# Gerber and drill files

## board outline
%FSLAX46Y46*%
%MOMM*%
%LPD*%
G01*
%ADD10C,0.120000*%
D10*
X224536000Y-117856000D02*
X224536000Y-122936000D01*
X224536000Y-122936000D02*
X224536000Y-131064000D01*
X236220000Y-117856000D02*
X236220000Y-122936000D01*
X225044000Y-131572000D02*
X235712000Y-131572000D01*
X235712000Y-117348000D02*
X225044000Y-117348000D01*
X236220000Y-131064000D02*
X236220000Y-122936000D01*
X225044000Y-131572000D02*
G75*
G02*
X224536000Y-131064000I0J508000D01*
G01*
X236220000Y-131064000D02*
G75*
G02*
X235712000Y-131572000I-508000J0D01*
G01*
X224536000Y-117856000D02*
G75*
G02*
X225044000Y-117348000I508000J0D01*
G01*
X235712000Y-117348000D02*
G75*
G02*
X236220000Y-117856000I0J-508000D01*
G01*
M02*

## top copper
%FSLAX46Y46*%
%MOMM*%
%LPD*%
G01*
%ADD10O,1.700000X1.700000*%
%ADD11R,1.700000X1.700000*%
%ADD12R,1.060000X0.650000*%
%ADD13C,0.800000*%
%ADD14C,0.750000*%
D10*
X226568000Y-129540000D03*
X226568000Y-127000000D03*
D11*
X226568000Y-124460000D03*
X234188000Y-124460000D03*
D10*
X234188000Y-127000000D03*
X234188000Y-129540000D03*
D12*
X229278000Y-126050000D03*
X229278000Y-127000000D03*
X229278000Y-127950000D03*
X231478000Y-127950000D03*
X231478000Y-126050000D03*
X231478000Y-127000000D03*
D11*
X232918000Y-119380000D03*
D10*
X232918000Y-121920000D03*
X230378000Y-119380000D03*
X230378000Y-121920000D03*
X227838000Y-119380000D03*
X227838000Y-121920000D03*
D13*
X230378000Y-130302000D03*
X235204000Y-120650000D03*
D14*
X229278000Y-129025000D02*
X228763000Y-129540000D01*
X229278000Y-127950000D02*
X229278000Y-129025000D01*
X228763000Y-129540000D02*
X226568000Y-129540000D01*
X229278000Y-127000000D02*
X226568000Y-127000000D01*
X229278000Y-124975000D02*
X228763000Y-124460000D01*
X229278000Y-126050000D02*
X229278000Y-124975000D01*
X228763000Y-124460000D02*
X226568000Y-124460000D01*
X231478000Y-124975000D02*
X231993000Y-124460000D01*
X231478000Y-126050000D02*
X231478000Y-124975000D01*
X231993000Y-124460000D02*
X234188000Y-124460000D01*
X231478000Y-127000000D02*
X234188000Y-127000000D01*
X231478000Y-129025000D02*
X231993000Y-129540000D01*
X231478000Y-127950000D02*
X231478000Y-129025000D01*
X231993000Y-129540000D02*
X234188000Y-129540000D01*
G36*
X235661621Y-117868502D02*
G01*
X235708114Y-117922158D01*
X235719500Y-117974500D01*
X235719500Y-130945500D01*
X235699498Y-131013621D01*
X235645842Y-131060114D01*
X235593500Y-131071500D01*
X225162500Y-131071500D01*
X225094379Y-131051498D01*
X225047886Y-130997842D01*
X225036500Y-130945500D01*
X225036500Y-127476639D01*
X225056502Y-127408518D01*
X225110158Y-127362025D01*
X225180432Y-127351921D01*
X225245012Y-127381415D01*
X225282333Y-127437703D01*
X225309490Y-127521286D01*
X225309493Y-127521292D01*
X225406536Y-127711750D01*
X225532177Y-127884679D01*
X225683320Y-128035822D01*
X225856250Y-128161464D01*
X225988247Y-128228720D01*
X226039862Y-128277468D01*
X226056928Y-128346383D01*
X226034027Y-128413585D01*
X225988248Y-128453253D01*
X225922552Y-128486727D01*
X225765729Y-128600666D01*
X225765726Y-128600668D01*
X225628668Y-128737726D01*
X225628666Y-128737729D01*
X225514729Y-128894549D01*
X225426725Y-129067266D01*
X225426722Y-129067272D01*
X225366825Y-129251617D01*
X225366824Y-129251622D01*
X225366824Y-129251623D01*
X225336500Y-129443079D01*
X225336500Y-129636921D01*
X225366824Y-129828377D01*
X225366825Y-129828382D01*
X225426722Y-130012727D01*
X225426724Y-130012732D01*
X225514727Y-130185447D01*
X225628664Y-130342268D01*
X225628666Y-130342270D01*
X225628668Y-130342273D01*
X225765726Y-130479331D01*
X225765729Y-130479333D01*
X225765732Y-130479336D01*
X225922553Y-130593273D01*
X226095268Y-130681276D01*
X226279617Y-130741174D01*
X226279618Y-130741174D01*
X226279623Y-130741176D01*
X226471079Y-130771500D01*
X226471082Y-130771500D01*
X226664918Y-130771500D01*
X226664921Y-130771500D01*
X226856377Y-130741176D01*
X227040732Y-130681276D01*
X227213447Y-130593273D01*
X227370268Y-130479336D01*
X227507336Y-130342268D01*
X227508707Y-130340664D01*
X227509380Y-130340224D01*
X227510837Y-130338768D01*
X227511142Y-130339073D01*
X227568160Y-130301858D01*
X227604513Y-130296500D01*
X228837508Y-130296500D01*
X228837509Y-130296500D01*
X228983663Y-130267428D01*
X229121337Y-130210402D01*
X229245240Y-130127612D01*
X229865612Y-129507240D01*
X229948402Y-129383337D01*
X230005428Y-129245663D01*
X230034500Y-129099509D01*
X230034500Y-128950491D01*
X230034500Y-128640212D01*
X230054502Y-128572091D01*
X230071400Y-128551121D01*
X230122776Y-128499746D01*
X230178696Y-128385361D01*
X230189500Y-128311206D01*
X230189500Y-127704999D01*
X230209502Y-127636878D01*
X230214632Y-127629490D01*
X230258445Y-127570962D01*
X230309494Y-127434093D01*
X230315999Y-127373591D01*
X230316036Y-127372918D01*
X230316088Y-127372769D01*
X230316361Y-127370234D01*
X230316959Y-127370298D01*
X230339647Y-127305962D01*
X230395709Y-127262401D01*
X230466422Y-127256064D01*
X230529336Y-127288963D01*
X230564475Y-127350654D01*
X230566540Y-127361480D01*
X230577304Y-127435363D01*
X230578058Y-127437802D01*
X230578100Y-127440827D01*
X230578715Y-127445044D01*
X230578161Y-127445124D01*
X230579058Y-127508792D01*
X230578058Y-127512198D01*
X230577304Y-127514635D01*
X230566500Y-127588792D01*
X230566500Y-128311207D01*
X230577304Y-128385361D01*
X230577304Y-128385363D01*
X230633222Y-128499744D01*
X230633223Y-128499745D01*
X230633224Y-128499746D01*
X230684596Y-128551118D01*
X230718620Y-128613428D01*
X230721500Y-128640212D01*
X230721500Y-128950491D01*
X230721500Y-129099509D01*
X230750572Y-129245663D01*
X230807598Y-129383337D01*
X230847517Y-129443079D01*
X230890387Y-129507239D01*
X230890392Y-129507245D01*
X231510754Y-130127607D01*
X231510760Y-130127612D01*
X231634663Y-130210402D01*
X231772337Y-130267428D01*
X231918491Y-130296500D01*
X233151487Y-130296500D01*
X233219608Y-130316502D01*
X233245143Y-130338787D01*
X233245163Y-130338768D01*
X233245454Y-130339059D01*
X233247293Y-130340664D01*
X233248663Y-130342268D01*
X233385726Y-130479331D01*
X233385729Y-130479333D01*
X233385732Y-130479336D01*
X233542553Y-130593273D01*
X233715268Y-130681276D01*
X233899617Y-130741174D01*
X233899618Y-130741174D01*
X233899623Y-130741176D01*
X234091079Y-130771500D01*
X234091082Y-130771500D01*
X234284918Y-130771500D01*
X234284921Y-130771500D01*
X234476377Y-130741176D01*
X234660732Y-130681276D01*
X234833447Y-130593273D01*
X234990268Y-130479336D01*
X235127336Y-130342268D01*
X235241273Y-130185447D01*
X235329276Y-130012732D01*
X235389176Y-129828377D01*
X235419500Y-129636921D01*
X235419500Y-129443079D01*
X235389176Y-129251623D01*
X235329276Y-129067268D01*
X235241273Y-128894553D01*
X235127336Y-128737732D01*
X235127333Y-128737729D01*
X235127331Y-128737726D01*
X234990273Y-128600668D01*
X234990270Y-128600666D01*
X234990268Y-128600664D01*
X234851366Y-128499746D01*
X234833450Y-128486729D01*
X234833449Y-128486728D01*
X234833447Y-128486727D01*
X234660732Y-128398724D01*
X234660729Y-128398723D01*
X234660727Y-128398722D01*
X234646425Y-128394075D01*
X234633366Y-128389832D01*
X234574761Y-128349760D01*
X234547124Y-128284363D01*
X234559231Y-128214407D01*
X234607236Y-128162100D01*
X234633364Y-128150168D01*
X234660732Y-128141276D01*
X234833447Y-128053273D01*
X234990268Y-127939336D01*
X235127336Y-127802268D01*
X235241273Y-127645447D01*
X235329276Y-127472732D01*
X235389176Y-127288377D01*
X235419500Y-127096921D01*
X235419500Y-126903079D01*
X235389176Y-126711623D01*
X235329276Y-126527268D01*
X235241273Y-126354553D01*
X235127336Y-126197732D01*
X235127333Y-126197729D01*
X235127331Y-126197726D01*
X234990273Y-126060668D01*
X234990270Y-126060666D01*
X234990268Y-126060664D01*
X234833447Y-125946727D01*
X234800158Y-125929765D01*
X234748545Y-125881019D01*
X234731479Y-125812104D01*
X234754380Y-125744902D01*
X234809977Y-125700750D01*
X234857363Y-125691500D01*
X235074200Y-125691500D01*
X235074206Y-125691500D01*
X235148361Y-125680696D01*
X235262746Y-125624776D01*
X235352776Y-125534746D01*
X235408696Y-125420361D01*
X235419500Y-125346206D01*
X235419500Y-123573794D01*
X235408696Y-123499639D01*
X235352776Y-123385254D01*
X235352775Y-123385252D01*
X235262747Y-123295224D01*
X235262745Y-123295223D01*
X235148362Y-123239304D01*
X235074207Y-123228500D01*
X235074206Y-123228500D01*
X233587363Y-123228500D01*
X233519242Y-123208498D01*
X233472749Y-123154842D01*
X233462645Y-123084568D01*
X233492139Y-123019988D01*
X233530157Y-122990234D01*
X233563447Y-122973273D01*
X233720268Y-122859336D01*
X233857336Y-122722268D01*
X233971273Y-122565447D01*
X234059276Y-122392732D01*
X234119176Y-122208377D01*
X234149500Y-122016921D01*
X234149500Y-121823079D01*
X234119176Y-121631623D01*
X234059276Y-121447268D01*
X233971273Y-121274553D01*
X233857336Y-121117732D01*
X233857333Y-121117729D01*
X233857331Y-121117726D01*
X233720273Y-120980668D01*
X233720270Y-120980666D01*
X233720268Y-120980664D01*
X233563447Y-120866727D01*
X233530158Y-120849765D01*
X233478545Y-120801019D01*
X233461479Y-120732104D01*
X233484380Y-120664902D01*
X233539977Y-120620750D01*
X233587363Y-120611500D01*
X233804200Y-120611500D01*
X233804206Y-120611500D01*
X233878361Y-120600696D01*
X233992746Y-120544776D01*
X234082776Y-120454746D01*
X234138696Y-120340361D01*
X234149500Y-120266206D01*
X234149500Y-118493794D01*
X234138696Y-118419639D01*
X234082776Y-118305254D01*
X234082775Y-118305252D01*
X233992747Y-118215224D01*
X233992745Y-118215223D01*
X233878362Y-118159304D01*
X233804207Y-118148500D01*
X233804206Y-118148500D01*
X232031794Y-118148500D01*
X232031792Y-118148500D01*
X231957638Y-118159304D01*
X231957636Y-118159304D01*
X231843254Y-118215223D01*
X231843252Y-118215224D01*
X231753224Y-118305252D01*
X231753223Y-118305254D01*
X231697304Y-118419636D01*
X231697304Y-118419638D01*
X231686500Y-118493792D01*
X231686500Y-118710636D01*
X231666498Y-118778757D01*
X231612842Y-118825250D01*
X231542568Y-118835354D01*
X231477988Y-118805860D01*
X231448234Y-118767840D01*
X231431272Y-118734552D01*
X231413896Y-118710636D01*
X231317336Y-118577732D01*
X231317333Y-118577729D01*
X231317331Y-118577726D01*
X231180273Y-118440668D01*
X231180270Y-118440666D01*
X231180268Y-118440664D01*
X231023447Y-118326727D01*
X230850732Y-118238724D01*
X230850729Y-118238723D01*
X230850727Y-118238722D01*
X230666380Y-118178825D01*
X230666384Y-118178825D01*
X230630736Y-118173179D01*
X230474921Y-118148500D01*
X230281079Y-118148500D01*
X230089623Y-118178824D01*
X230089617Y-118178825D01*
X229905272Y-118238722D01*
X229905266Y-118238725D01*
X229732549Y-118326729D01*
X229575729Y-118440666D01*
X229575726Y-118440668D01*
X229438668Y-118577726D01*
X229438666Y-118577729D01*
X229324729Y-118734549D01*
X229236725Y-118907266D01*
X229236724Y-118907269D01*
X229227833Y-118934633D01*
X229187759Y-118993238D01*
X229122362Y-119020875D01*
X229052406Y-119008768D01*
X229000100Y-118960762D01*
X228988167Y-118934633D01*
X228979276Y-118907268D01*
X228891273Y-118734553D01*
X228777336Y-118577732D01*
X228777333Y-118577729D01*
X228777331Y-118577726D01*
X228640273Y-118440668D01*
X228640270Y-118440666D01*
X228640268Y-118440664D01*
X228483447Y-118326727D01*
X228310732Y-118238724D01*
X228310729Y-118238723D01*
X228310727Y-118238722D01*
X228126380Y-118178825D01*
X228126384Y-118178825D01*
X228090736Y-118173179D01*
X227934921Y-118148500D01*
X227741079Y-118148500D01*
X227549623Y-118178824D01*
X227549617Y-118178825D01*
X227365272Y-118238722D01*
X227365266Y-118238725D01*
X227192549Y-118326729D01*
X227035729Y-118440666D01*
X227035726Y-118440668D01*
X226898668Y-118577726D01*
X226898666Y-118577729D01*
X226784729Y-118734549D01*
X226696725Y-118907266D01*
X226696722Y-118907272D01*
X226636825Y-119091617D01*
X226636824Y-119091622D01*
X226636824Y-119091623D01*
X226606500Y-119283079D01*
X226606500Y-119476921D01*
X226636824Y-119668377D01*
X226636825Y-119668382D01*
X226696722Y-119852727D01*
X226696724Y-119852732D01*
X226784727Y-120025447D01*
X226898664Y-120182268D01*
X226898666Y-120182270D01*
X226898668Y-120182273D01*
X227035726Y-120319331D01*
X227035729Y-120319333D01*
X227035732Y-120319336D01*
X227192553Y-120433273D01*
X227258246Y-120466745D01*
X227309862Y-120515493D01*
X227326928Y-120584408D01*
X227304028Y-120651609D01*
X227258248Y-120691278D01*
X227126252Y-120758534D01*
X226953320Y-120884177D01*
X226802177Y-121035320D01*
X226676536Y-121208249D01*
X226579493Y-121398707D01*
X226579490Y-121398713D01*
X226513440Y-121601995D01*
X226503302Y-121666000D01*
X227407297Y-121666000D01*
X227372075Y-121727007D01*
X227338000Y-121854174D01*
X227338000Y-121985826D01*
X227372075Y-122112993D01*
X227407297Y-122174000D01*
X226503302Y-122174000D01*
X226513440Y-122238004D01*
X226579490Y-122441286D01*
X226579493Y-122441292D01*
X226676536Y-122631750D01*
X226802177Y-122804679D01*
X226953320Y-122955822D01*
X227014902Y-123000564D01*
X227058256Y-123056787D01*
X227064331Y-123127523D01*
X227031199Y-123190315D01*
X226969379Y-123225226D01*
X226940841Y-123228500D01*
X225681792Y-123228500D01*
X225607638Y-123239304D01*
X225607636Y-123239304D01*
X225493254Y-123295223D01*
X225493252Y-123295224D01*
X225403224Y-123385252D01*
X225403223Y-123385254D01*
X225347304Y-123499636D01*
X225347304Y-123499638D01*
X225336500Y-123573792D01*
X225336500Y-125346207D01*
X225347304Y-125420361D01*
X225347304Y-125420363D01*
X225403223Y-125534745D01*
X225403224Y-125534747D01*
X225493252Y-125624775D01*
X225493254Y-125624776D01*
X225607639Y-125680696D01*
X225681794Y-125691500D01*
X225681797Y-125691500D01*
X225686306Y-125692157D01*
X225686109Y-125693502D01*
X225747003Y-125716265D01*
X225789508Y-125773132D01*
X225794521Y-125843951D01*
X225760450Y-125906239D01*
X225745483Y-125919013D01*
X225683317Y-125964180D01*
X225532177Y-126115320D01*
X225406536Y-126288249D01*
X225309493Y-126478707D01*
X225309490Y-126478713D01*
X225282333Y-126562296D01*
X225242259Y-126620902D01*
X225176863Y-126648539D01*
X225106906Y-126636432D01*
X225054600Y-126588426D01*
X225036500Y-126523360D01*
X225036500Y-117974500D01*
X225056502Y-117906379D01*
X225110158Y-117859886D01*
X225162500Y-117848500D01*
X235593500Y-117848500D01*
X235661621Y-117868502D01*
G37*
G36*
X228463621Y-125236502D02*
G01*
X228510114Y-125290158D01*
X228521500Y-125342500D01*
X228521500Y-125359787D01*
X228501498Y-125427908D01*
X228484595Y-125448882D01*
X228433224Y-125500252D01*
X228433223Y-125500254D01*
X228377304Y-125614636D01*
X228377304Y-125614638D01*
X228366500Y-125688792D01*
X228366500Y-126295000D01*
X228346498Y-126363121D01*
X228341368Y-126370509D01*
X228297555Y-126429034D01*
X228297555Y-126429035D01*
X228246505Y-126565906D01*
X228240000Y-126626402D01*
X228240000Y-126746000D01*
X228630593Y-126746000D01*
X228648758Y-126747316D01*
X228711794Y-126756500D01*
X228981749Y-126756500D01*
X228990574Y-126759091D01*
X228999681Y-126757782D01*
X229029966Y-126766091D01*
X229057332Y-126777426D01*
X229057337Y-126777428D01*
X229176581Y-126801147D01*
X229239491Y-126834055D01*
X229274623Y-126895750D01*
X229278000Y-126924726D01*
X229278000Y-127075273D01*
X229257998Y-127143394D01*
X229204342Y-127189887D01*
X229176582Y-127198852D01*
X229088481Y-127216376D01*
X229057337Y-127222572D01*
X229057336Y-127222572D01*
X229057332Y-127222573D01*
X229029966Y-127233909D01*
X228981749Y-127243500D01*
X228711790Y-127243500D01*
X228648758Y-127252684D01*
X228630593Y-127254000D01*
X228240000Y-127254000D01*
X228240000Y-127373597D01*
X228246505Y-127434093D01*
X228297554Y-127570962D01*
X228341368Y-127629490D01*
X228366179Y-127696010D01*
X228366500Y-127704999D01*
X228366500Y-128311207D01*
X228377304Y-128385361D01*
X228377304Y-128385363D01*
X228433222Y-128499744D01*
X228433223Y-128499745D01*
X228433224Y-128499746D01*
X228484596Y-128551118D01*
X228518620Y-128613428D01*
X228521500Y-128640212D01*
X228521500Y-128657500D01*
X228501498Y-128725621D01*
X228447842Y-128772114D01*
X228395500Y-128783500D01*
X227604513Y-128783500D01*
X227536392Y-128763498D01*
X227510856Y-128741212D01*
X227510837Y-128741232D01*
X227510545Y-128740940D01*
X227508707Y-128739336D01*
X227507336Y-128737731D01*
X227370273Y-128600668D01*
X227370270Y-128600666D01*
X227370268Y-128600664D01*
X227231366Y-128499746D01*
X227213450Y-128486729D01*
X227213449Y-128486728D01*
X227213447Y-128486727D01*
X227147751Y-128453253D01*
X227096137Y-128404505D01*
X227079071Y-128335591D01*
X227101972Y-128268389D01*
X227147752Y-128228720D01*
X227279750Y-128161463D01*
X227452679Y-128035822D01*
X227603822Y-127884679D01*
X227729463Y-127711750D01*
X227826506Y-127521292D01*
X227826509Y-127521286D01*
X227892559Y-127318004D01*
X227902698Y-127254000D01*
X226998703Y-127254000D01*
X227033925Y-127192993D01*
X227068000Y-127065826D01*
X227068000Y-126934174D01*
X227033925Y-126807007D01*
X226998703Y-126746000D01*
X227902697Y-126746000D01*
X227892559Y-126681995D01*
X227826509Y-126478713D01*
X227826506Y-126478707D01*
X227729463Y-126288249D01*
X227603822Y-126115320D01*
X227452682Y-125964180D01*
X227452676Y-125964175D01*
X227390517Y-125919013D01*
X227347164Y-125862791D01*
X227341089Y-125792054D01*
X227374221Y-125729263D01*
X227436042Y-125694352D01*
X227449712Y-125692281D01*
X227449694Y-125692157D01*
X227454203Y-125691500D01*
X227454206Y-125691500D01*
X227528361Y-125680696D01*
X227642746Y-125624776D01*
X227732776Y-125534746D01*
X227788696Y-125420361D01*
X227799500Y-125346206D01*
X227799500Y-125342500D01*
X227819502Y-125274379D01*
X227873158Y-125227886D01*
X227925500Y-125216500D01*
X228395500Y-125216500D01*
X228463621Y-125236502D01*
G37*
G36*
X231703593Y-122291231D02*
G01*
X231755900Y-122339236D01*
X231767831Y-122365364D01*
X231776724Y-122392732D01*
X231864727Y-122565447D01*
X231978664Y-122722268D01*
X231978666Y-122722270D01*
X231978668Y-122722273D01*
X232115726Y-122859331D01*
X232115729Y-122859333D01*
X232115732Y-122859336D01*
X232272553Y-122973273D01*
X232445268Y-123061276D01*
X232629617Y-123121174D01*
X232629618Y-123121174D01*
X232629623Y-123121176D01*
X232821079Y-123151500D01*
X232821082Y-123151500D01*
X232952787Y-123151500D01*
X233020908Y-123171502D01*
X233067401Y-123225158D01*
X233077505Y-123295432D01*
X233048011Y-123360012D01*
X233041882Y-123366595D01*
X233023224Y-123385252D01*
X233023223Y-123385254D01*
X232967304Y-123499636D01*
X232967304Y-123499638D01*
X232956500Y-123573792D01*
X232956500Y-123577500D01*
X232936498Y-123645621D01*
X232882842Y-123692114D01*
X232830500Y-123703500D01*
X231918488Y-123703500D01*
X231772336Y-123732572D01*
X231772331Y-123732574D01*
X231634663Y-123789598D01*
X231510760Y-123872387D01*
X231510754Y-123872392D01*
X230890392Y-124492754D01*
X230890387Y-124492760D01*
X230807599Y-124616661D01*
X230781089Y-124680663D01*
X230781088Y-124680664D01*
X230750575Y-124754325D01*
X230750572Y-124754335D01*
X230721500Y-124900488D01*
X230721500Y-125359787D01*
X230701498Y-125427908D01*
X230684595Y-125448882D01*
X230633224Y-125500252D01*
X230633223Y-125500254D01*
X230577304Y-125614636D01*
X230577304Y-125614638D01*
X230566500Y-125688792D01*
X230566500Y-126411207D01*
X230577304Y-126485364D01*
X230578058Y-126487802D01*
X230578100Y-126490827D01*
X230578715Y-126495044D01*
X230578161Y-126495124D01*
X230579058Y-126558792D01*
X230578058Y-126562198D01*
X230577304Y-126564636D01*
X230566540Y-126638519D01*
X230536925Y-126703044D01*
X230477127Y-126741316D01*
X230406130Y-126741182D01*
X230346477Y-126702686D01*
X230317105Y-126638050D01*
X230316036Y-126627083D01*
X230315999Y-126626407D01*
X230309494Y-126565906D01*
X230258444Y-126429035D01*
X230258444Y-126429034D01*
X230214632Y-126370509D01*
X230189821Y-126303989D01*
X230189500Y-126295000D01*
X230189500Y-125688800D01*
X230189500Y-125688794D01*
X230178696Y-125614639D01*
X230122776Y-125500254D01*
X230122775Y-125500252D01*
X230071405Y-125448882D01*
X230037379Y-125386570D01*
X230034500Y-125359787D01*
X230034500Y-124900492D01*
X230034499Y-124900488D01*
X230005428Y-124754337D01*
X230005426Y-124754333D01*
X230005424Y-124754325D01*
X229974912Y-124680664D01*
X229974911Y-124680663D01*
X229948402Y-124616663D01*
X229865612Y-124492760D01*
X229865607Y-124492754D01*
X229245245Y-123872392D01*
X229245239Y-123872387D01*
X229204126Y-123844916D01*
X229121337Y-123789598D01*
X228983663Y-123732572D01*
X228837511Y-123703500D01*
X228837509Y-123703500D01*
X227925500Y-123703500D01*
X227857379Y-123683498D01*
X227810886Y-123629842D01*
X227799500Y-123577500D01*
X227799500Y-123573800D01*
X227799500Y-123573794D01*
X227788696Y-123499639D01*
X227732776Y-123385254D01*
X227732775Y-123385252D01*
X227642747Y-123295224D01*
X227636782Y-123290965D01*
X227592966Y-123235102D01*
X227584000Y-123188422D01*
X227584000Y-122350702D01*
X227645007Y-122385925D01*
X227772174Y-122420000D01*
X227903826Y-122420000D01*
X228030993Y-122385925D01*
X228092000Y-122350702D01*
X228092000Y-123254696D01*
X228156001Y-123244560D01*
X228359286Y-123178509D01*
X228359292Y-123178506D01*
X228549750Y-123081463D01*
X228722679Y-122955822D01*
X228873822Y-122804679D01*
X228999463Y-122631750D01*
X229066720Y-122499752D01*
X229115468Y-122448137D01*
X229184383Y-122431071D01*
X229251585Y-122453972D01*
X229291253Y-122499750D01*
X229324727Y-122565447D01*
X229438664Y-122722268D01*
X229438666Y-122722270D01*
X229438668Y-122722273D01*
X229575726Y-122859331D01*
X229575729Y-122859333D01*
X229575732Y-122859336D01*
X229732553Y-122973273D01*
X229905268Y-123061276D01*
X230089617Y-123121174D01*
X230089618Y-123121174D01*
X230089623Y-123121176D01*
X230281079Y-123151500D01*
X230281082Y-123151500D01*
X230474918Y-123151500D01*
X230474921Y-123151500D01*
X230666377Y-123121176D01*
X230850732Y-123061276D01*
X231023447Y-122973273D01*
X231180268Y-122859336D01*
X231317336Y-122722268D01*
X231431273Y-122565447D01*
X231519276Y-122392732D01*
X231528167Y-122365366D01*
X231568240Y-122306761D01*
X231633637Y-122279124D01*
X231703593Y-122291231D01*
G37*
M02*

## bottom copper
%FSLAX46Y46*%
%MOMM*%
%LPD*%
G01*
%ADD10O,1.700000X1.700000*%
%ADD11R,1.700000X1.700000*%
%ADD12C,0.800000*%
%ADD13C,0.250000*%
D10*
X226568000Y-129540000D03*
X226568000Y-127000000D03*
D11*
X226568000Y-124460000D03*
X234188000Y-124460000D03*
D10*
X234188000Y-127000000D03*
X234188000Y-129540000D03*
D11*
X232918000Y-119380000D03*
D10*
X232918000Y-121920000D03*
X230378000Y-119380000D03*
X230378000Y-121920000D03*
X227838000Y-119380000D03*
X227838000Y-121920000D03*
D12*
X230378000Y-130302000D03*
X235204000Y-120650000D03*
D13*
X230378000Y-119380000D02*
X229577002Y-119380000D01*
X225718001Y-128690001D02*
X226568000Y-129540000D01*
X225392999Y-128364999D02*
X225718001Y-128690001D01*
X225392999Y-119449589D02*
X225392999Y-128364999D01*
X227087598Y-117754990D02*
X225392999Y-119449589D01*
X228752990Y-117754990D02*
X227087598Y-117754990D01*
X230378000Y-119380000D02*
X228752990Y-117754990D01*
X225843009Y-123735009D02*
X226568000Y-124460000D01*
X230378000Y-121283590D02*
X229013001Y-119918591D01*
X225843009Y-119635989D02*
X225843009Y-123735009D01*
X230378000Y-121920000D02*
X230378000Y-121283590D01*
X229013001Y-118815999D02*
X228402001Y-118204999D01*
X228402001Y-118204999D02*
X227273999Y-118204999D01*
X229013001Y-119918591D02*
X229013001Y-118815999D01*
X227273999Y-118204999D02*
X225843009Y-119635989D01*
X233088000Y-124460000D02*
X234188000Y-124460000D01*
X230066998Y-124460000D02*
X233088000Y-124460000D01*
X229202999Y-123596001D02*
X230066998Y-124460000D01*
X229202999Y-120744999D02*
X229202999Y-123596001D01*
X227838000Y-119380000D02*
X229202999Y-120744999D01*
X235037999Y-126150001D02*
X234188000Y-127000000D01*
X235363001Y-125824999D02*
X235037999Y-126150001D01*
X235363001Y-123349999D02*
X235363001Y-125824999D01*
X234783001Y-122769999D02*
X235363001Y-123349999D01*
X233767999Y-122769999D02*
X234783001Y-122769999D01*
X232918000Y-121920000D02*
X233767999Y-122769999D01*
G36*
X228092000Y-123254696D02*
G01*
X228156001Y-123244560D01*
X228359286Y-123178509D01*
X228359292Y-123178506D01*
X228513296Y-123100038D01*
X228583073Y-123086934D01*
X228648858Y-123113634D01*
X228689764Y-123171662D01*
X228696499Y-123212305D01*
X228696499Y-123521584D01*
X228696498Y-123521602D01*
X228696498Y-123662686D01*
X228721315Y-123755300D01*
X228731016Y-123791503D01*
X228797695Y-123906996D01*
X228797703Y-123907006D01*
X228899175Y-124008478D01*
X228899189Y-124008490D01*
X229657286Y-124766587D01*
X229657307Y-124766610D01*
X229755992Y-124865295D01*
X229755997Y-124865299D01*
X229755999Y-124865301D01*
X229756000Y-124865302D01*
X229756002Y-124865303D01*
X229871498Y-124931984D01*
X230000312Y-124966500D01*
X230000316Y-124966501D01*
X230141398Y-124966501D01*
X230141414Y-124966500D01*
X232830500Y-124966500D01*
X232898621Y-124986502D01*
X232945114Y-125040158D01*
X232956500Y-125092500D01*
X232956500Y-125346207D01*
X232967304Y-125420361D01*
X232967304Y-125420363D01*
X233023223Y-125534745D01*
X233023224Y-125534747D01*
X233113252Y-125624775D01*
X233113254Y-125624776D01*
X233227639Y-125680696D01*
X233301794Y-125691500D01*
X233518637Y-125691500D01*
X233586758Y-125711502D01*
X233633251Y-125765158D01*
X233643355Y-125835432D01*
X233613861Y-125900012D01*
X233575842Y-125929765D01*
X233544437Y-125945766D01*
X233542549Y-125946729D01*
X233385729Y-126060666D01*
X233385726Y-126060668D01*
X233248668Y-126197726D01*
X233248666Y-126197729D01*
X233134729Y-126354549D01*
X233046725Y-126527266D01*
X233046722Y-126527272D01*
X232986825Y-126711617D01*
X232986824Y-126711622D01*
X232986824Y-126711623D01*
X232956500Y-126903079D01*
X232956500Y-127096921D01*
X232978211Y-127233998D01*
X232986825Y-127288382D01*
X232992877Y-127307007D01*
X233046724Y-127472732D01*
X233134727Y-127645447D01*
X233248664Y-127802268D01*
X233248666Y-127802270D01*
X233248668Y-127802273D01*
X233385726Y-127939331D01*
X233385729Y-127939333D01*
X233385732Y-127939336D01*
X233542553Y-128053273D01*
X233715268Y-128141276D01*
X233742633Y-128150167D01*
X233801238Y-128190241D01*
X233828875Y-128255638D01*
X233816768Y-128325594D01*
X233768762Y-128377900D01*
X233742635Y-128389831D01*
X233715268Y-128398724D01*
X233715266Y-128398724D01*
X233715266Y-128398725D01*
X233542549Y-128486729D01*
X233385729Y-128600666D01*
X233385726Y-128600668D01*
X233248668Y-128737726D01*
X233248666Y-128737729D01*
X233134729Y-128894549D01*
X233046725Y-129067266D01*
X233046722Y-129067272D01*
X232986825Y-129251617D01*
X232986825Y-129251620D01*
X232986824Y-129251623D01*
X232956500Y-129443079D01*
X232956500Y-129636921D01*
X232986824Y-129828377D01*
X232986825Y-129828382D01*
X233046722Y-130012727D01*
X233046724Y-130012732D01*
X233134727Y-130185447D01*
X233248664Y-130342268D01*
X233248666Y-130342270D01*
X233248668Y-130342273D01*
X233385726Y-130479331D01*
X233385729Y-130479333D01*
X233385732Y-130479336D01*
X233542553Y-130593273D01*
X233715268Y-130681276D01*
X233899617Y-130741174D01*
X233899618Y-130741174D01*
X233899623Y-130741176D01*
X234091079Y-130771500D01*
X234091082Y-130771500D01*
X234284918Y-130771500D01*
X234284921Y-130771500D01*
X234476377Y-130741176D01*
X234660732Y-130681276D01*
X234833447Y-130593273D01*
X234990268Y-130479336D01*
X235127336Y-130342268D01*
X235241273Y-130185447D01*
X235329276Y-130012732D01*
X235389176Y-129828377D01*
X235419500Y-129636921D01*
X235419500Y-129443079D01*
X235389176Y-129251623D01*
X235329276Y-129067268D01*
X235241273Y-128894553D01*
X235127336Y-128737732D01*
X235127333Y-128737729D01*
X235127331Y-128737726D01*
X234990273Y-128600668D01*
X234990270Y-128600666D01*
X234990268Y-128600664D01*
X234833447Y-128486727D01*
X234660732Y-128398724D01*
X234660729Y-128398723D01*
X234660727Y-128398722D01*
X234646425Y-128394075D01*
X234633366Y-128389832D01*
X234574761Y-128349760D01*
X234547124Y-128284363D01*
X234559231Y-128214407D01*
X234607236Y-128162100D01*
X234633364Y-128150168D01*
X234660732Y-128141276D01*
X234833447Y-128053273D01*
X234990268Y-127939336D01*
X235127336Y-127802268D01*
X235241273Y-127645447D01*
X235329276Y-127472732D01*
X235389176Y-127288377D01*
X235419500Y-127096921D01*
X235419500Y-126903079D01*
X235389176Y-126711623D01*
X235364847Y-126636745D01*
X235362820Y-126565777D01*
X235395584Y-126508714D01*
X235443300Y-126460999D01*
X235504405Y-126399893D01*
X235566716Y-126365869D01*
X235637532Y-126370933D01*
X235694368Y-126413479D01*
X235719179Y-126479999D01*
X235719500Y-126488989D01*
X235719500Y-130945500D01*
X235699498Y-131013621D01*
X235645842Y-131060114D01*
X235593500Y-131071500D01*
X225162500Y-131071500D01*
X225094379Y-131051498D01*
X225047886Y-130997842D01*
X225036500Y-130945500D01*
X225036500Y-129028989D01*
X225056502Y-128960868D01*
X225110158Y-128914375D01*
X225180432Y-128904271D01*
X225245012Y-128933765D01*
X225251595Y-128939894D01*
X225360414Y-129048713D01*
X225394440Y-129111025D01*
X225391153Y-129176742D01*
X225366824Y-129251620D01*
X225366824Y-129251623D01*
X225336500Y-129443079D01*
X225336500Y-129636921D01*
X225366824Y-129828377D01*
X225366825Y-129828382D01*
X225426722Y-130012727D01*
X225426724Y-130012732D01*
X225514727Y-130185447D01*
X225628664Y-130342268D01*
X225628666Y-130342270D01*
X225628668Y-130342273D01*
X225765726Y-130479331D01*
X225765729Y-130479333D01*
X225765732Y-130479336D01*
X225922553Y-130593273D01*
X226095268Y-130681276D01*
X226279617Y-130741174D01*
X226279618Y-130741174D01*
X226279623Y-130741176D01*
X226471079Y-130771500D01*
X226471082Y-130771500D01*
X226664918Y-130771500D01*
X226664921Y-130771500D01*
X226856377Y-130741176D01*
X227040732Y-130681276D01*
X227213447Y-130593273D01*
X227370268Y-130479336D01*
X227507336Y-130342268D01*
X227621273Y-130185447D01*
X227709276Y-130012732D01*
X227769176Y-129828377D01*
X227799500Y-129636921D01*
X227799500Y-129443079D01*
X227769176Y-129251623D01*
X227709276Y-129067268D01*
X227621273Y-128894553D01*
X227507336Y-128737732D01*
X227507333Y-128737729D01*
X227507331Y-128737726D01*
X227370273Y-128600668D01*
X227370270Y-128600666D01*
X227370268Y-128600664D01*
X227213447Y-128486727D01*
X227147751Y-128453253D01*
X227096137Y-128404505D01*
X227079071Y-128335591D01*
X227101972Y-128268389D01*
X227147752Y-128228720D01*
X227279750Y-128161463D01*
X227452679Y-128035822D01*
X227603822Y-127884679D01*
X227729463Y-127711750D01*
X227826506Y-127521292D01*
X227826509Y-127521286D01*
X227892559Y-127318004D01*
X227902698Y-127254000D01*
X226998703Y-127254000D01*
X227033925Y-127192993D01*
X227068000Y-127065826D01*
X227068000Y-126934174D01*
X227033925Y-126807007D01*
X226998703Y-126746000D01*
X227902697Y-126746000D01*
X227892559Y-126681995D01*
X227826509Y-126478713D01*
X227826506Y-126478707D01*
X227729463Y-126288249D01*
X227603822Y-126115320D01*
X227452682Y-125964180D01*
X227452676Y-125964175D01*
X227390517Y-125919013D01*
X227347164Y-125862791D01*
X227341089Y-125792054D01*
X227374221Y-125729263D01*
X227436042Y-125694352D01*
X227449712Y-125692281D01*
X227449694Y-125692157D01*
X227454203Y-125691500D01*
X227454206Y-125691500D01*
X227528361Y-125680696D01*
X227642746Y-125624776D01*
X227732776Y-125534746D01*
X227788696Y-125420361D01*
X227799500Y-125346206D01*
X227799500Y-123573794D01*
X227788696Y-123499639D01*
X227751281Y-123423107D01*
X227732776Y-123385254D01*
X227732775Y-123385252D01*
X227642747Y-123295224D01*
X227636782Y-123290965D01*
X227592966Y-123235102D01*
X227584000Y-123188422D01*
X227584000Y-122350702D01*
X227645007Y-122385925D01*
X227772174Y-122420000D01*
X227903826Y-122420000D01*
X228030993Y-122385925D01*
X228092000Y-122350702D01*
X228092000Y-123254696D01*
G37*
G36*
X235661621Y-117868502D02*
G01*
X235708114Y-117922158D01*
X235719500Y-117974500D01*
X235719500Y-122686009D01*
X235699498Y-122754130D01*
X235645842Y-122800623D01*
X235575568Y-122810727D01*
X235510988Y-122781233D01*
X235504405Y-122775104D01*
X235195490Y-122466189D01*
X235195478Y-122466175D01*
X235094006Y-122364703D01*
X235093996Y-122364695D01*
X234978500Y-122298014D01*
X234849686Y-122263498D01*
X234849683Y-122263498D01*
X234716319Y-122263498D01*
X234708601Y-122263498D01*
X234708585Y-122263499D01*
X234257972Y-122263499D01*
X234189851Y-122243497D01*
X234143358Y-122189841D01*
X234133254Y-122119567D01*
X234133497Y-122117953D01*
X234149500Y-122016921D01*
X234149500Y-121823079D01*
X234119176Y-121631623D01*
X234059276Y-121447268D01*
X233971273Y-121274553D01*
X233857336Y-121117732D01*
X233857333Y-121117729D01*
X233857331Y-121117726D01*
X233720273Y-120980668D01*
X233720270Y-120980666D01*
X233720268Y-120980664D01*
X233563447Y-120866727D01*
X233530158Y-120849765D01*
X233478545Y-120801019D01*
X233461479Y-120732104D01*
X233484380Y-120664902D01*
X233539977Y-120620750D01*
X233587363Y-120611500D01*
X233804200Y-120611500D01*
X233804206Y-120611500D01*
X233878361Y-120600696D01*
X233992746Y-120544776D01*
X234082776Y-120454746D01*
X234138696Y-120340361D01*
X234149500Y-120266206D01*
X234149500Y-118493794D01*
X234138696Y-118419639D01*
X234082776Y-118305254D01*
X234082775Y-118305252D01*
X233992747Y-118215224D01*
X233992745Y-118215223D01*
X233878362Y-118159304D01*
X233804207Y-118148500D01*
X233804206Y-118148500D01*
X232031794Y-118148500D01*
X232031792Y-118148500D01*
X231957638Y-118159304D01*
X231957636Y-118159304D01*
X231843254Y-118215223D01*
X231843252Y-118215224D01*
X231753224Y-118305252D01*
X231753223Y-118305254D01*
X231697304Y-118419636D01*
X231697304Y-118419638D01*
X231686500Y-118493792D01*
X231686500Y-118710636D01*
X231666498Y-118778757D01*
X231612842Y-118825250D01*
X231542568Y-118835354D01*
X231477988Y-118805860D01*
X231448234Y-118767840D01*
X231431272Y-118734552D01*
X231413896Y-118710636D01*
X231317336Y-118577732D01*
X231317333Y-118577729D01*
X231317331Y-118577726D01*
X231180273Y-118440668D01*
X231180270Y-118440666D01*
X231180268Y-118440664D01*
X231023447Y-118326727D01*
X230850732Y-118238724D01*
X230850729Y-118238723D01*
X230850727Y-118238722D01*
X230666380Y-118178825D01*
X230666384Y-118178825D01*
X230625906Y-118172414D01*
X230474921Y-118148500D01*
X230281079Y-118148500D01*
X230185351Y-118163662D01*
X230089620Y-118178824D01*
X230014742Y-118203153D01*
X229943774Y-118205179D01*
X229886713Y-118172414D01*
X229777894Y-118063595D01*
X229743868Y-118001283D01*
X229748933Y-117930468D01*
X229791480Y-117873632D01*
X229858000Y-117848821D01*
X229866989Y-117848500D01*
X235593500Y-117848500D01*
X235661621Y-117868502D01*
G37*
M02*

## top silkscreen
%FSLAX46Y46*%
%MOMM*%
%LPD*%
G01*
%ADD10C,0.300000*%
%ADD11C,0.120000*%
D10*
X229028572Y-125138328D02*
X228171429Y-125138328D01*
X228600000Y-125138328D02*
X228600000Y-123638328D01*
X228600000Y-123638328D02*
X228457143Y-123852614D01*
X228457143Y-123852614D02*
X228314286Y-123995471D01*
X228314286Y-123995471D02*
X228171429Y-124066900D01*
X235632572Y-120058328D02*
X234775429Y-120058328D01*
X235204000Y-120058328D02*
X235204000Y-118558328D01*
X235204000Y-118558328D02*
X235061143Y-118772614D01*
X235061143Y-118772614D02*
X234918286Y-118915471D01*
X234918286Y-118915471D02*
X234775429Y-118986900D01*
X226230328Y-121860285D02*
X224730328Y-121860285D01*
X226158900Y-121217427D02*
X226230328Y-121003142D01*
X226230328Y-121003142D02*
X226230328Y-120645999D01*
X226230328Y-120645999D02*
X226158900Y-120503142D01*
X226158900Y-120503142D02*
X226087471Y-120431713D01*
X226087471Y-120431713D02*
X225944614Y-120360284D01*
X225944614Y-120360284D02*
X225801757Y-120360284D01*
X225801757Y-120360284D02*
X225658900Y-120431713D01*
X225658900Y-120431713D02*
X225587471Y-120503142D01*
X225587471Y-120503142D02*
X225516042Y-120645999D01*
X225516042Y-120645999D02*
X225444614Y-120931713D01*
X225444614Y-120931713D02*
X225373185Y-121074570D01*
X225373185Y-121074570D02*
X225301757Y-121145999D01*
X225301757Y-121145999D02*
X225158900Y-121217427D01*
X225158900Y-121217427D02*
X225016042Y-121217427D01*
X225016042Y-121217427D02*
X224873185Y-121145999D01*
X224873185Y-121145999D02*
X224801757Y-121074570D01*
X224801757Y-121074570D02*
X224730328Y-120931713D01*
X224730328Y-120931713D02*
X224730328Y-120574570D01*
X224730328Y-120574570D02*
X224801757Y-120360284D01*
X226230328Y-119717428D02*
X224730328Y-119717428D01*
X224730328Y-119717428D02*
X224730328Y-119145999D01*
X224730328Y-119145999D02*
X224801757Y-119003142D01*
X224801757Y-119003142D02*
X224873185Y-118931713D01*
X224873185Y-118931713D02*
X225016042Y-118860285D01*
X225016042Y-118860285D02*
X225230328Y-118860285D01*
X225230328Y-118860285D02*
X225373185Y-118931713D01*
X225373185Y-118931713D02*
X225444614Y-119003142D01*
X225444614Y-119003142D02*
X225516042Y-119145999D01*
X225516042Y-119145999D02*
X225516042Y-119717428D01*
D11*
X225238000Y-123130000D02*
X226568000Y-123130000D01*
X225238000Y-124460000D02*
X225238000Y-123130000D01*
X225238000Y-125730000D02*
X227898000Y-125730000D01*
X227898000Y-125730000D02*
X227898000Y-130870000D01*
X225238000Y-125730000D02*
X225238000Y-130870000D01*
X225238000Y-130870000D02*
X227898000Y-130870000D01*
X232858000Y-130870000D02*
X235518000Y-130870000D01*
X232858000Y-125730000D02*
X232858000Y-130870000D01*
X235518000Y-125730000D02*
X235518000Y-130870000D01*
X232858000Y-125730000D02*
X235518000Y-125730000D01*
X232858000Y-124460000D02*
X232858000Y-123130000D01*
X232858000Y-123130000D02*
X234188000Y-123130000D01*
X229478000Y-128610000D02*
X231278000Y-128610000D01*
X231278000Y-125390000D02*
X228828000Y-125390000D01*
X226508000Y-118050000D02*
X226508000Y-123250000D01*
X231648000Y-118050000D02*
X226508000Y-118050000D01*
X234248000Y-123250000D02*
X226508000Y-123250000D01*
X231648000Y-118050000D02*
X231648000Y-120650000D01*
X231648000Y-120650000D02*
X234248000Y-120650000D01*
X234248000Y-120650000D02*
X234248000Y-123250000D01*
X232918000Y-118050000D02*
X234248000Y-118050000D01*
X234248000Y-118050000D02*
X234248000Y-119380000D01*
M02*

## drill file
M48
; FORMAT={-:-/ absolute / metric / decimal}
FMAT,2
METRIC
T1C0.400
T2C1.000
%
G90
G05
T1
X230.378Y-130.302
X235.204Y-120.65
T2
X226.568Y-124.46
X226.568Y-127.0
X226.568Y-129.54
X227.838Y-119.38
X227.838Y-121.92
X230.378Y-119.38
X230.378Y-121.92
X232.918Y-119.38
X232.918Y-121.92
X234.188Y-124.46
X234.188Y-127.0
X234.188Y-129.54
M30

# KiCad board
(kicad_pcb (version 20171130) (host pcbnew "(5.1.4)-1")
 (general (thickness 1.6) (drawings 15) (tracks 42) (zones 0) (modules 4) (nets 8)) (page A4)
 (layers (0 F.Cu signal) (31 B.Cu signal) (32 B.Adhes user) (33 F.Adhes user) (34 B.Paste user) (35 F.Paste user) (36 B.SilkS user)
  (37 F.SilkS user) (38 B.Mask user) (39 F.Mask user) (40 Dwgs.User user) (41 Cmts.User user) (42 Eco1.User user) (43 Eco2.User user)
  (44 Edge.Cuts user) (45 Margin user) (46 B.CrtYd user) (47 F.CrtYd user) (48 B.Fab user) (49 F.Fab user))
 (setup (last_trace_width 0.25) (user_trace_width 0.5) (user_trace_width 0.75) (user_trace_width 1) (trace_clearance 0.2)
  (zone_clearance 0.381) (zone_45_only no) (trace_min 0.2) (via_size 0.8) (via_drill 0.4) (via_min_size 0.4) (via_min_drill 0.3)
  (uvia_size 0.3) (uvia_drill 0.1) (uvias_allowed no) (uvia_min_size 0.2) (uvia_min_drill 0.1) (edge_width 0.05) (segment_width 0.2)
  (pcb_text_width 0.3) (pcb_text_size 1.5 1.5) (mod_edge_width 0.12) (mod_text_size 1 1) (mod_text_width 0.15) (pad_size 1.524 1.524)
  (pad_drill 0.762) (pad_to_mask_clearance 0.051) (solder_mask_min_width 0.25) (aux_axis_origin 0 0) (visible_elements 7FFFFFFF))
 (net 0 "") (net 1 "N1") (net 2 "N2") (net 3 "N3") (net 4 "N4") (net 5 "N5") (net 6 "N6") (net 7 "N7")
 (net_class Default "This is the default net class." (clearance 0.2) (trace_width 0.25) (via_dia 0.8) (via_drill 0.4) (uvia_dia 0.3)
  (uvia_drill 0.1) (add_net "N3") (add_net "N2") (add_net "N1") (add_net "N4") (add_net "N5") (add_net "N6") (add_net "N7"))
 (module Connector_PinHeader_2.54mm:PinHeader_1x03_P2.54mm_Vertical (layer F.Cu) (at 226.568 124.46)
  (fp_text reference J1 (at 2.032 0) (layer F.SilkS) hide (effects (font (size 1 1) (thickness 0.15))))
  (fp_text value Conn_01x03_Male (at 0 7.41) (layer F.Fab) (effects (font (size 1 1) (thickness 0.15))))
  (fp_line (start -1.33 -1.33) (end 0 -1.33) (layer F.SilkS) (width 0.12))
  (fp_line (start -1.33 0) (end -1.33 -1.33) (layer F.SilkS) (width 0.12))
  (fp_line (start -1.33 1.27) (end 1.33 1.27) (layer F.SilkS) (width 0.12))
  (fp_line (start 1.33 1.27) (end 1.33 6.41) (layer F.SilkS) (width 0.12))
  (fp_line (start -1.33 1.27) (end -1.33 6.41) (layer F.SilkS) (width 0.12))
  (fp_line (start -1.33 6.41) (end 1.33 6.41) (layer F.SilkS) (width 0.12))
  (pad 3 thru_hole oval (at 0 5.08) (size 1.7 1.7) (drill 1) (layers *.Cu *.Mask) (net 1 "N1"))
  (pad 2 thru_hole oval (at 0 2.54) (size 1.7 1.7) (drill 1) (layers *.Cu *.Mask) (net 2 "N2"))
  (pad 1 thru_hole rect (at 0 0) (size 1.7 1.7) (drill 1) (layers *.Cu *.Mask) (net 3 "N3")))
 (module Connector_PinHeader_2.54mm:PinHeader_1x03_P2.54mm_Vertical (layer F.Cu) (at 234.188 124.46)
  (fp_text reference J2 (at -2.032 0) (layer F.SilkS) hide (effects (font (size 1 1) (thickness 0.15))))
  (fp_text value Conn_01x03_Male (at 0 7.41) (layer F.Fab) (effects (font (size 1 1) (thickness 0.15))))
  (fp_line (start -1.33 6.41) (end 1.33 6.41) (layer F.SilkS) (width 0.12))
  (fp_line (start -1.33 1.27) (end -1.33 6.41) (layer F.SilkS) (width 0.12))
  (fp_line (start 1.33 1.27) (end 1.33 6.41) (layer F.SilkS) (width 0.12))
  (fp_line (start -1.33 1.27) (end 1.33 1.27) (layer F.SilkS) (width 0.12))
  (fp_line (start -1.33 0) (end -1.33 -1.33) (layer F.SilkS) (width 0.12))
  (fp_line (start -1.33 -1.33) (end 0 -1.33) (layer F.SilkS) (width 0.12))
  (pad 1 thru_hole rect (at 0 0) (size 1.7 1.7) (drill 1) (layers *.Cu *.Mask) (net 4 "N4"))
  (pad 2 thru_hole oval (at 0 2.54) (size 1.7 1.7) (drill 1) (layers *.Cu *.Mask) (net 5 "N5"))
  (pad 3 thru_hole oval (at 0 5.08) (size 1.7 1.7) (drill 1) (layers *.Cu *.Mask) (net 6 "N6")))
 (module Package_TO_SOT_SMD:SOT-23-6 (layer F.Cu) (at 230.378 127)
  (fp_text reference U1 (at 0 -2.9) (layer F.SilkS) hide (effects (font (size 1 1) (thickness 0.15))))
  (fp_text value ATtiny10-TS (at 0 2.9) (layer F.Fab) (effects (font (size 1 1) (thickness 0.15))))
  (fp_line (start -0.9 1.61) (end 0.9 1.61) (layer F.SilkS) (width 0.12))
  (fp_line (start 0.9 -1.61) (end -1.55 -1.61) (layer F.SilkS) (width 0.12))
  (pad 1 smd rect (at -1.1 -0.95) (size 1.06 0.65) (layers F.Cu F.Paste F.Mask) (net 3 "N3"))
  (pad 2 smd rect (at -1.1 0) (size 1.06 0.65) (layers F.Cu F.Paste F.Mask) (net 2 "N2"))
  (pad 3 smd rect (at -1.1 0.95) (size 1.06 0.65) (layers F.Cu F.Paste F.Mask) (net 1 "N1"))
  (pad 4 smd rect (at 1.1 0.95) (size 1.06 0.65) (layers F.Cu F.Paste F.Mask) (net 6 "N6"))
  (pad 6 smd rect (at 1.1 -0.95) (size 1.06 0.65) (layers F.Cu F.Paste F.Mask) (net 4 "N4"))
  (pad 5 smd rect (at 1.1 0) (size 1.06 0.65) (layers F.Cu F.Paste F.Mask) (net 5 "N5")))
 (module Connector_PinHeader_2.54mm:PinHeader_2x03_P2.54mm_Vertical (layer F.Cu) (at 232.918 119.38 270)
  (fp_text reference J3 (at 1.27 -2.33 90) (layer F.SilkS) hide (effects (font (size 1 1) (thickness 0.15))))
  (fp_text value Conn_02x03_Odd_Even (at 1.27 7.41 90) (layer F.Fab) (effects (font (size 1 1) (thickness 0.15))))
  (fp_line (start -1.33 6.41) (end 3.87 6.41) (layer F.SilkS) (width 0.12))
  (fp_line (start -1.33 1.27) (end -1.33 6.41) (layer F.SilkS) (width 0.12))
  (fp_line (start 3.87 -1.33) (end 3.87 6.41) (layer F.SilkS) (width 0.12))
  (fp_line (start -1.33 1.27) (end 1.27 1.27) (layer F.SilkS) (width 0.12))
  (fp_line (start 1.27 1.27) (end 1.27 -1.33) (layer F.SilkS) (width 0.12))
  (fp_line (start 1.27 -1.33) (end 3.87 -1.33) (layer F.SilkS) (width 0.12))
  (fp_line (start -1.33 0) (end -1.33 -1.33) (layer F.SilkS) (width 0.12))
  (fp_line (start -1.33 -1.33) (end 0 -1.33) (layer F.SilkS) (width 0.12))
  (pad 1 thru_hole rect (at 0 0 270) (size 1.7 1.7) (drill 1) (layers *.Cu *.Mask) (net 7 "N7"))
  (pad 2 thru_hole oval (at 2.54 0 270) (size 1.7 1.7) (drill 1) (layers *.Cu *.Mask) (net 5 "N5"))
  (pad 3 thru_hole oval (at 0 2.54 270) (size 1.7 1.7) (drill 1) (layers *.Cu *.Mask) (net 1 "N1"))
  (pad 4 thru_hole oval (at 2.54 2.54 270) (size 1.7 1.7) (drill 1) (layers *.Cu *.Mask) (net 3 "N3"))
  (pad 5 thru_hole oval (at 0 5.08 270) (size 1.7 1.7) (drill 1) (layers *.Cu *.Mask) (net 4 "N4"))
  (pad 6 thru_hole oval (at 2.54 5.08 270) (size 1.7 1.7) (drill 1) (layers *.Cu *.Mask) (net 2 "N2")))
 (gr_line (start 224.536 117.856) (end 224.536 122.936) (layer Edge.Cuts) (width 0.12))
 (gr_line (start 224.536 122.936) (end 224.536 131.064) (layer Edge.Cuts) (width 0.12))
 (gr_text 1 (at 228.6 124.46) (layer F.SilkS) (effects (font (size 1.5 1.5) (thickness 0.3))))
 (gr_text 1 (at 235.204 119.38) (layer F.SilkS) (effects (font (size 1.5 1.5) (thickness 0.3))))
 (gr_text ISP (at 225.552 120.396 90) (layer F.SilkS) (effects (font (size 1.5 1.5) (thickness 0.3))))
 (gr_line (start 236.22 117.856) (end 236.22 122.936) (layer Edge.Cuts) (width 0.12))
 (gr_line (start 225.044 131.572) (end 235.712 131.572) (layer Edge.Cuts) (width 0.12))
 (gr_line (start 235.712 117.348) (end 225.044 117.348) (layer Edge.Cuts) (width 0.12))
 (gr_line (start 236.22 131.064) (end 236.22 122.936) (layer Edge.Cuts) (width 0.12))
 (gr_arc (start 225.044 131.064) (end 224.536 131.064) (angle -90) (layer Edge.Cuts) (width 0.12))
 (gr_arc (start 235.712 131.064) (end 235.712 131.572) (angle -90) (layer Edge.Cuts) (width 0.12))
 (gr_arc (start 225.044 117.856) (end 225.044 117.348) (angle -90) (layer Edge.Cuts) (width 0.12))
 (gr_arc (start 235.712 117.856) (end 236.22 117.856) (angle -90) (layer Edge.Cuts) (width 0.12))
 (segment (start 229.278 129.025) (end 228.763 129.54) (width 0.75) (layer F.Cu) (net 1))
 (segment (start 229.278 127.95) (end 229.278 129.025) (width 0.75) (layer F.Cu) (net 1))
 (segment (start 228.763 129.54) (end 226.568 129.54) (width 0.75) (layer F.Cu) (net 1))
 (segment (start 230.378 119.38) (end 229.577002 119.38) (width 0.25) (layer B.Cu) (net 1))
 (segment (start 225.718001 128.690001) (end 226.568 129.54) (width 0.25) (layer B.Cu) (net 1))
 (segment (start 225.392999 128.364999) (end 225.718001 128.690001) (width 0.25) (layer B.Cu) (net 1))
 (segment (start 225.392999 119.449589) (end 225.392999 128.364999) (width 0.25) (layer B.Cu) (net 1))
 (segment (start 227.087598 117.75499) (end 225.392999 119.449589) (width 0.25) (layer B.Cu) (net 1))
 (segment (start 228.75299 117.75499) (end 227.087598 117.75499) (width 0.25) (layer B.Cu) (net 1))
 (segment (start 230.378 119.38) (end 228.75299 117.75499) (width 0.25) (layer B.Cu) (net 1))
 (segment (start 229.278 127) (end 226.568 127) (width 0.75) (layer F.Cu) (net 2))
 (via (at 230.378 130.302) (size 0.8) (drill 0.4) (layers F.Cu B.Cu) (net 2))
 (via (at 235.204 120.65) (size 0.8) (drill 0.4) (layers F.Cu B.Cu) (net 2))
 (segment (start 229.278 124.975) (end 228.763 124.46) (width 0.75) (layer F.Cu) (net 3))
 (segment (start 229.278 126.05) (end 229.278 124.975) (width 0.75) (layer F.Cu) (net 3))
 (segment (start 228.763 124.46) (end 226.568 124.46) (width 0.75) (layer F.Cu) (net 3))
 (segment (start 225.843009 123.735009) (end 226.568 124.46) (width 0.25) (layer B.Cu) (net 3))
 (segment (start 230.378 121.28359) (end 229.013001 119.918591) (width 0.25) (layer B.Cu) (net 3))
 (segment (start 225.843009 119.635989) (end 225.843009 123.735009) (width 0.25) (layer B.Cu) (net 3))
 (segment (start 230.378 121.92) (end 230.378 121.28359) (width 0.25) (layer B.Cu) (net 3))
 (segment (start 229.013001 118.815999) (end 228.402001 118.204999) (width 0.25) (layer B.Cu) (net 3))
 (segment (start 228.402001 118.204999) (end 227.273999 118.204999) (width 0.25) (layer B.Cu) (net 3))
 (segment (start 229.013001 119.918591) (end 229.013001 118.815999) (width 0.25) (layer B.Cu) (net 3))
 (segment (start 227.273999 118.204999) (end 225.843009 119.635989) (width 0.25) (layer B.Cu) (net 3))
 (segment (start 231.478 124.975) (end 231.993 124.46) (width 0.75) (layer F.Cu) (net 4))
 (segment (start 231.478 126.05) (end 231.478 124.975) (width 0.75) (layer F.Cu) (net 4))
 (segment (start 231.993 124.46) (end 234.188 124.46) (width 0.75) (layer F.Cu) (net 4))
 (segment (start 233.088 124.46) (end 234.188 124.46) (width 0.25) (layer B.Cu) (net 4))
 (segment (start 230.066998 124.46) (end 233.088 124.46) (width 0.25) (layer B.Cu) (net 4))
 (segment (start 229.202999 123.596001) (end 230.066998 124.46) (width 0.25) (layer B.Cu) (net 4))
 (segment (start 229.202999 120.744999) (end 229.202999 123.596001) (width 0.25) (layer B.Cu) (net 4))
 (segment (start 227.838 119.38) (end 229.202999 120.744999) (width 0.25) (layer B.Cu) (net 4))
 (segment (start 231.478 127) (end 234.188 127) (width 0.75) (layer F.Cu) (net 5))
 (segment (start 235.037999 126.150001) (end 234.188 127) (width 0.25) (layer B.Cu) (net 5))
 (segment (start 235.363001 125.824999) (end 235.037999 126.150001) (width 0.25) (layer B.Cu) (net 5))
 (segment (start 235.363001 123.349999) (end 235.363001 125.824999) (width 0.25) (layer B.Cu) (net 5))
 (segment (start 234.783001 122.769999) (end 235.363001 123.349999) (width 0.25) (layer B.Cu) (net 5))
 (segment (start 233.767999 122.769999) (end 234.783001 122.769999) (width 0.25) (layer B.Cu) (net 5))
 (segment (start 232.918 121.92) (end 233.767999 122.769999) (width 0.25) (layer B.Cu) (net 5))
 (segment (start 231.478 129.025) (end 231.993 129.54) (width 0.75) (layer F.Cu) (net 6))
 (segment (start 231.478 127.95) (end 231.478 129.025) (width 0.75) (layer F.Cu) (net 6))
 (segment (start 231.993 129.54) (end 234.188 129.54) (width 0.75) (layer F.Cu) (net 6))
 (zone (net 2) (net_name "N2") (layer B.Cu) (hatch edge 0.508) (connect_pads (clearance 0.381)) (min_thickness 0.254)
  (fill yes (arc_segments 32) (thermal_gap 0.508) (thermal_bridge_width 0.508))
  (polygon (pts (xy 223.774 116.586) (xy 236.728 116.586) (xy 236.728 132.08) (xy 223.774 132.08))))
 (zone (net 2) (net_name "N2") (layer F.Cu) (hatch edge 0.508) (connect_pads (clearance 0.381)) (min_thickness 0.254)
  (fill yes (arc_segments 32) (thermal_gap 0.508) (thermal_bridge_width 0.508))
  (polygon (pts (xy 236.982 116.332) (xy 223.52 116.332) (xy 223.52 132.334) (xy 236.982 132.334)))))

